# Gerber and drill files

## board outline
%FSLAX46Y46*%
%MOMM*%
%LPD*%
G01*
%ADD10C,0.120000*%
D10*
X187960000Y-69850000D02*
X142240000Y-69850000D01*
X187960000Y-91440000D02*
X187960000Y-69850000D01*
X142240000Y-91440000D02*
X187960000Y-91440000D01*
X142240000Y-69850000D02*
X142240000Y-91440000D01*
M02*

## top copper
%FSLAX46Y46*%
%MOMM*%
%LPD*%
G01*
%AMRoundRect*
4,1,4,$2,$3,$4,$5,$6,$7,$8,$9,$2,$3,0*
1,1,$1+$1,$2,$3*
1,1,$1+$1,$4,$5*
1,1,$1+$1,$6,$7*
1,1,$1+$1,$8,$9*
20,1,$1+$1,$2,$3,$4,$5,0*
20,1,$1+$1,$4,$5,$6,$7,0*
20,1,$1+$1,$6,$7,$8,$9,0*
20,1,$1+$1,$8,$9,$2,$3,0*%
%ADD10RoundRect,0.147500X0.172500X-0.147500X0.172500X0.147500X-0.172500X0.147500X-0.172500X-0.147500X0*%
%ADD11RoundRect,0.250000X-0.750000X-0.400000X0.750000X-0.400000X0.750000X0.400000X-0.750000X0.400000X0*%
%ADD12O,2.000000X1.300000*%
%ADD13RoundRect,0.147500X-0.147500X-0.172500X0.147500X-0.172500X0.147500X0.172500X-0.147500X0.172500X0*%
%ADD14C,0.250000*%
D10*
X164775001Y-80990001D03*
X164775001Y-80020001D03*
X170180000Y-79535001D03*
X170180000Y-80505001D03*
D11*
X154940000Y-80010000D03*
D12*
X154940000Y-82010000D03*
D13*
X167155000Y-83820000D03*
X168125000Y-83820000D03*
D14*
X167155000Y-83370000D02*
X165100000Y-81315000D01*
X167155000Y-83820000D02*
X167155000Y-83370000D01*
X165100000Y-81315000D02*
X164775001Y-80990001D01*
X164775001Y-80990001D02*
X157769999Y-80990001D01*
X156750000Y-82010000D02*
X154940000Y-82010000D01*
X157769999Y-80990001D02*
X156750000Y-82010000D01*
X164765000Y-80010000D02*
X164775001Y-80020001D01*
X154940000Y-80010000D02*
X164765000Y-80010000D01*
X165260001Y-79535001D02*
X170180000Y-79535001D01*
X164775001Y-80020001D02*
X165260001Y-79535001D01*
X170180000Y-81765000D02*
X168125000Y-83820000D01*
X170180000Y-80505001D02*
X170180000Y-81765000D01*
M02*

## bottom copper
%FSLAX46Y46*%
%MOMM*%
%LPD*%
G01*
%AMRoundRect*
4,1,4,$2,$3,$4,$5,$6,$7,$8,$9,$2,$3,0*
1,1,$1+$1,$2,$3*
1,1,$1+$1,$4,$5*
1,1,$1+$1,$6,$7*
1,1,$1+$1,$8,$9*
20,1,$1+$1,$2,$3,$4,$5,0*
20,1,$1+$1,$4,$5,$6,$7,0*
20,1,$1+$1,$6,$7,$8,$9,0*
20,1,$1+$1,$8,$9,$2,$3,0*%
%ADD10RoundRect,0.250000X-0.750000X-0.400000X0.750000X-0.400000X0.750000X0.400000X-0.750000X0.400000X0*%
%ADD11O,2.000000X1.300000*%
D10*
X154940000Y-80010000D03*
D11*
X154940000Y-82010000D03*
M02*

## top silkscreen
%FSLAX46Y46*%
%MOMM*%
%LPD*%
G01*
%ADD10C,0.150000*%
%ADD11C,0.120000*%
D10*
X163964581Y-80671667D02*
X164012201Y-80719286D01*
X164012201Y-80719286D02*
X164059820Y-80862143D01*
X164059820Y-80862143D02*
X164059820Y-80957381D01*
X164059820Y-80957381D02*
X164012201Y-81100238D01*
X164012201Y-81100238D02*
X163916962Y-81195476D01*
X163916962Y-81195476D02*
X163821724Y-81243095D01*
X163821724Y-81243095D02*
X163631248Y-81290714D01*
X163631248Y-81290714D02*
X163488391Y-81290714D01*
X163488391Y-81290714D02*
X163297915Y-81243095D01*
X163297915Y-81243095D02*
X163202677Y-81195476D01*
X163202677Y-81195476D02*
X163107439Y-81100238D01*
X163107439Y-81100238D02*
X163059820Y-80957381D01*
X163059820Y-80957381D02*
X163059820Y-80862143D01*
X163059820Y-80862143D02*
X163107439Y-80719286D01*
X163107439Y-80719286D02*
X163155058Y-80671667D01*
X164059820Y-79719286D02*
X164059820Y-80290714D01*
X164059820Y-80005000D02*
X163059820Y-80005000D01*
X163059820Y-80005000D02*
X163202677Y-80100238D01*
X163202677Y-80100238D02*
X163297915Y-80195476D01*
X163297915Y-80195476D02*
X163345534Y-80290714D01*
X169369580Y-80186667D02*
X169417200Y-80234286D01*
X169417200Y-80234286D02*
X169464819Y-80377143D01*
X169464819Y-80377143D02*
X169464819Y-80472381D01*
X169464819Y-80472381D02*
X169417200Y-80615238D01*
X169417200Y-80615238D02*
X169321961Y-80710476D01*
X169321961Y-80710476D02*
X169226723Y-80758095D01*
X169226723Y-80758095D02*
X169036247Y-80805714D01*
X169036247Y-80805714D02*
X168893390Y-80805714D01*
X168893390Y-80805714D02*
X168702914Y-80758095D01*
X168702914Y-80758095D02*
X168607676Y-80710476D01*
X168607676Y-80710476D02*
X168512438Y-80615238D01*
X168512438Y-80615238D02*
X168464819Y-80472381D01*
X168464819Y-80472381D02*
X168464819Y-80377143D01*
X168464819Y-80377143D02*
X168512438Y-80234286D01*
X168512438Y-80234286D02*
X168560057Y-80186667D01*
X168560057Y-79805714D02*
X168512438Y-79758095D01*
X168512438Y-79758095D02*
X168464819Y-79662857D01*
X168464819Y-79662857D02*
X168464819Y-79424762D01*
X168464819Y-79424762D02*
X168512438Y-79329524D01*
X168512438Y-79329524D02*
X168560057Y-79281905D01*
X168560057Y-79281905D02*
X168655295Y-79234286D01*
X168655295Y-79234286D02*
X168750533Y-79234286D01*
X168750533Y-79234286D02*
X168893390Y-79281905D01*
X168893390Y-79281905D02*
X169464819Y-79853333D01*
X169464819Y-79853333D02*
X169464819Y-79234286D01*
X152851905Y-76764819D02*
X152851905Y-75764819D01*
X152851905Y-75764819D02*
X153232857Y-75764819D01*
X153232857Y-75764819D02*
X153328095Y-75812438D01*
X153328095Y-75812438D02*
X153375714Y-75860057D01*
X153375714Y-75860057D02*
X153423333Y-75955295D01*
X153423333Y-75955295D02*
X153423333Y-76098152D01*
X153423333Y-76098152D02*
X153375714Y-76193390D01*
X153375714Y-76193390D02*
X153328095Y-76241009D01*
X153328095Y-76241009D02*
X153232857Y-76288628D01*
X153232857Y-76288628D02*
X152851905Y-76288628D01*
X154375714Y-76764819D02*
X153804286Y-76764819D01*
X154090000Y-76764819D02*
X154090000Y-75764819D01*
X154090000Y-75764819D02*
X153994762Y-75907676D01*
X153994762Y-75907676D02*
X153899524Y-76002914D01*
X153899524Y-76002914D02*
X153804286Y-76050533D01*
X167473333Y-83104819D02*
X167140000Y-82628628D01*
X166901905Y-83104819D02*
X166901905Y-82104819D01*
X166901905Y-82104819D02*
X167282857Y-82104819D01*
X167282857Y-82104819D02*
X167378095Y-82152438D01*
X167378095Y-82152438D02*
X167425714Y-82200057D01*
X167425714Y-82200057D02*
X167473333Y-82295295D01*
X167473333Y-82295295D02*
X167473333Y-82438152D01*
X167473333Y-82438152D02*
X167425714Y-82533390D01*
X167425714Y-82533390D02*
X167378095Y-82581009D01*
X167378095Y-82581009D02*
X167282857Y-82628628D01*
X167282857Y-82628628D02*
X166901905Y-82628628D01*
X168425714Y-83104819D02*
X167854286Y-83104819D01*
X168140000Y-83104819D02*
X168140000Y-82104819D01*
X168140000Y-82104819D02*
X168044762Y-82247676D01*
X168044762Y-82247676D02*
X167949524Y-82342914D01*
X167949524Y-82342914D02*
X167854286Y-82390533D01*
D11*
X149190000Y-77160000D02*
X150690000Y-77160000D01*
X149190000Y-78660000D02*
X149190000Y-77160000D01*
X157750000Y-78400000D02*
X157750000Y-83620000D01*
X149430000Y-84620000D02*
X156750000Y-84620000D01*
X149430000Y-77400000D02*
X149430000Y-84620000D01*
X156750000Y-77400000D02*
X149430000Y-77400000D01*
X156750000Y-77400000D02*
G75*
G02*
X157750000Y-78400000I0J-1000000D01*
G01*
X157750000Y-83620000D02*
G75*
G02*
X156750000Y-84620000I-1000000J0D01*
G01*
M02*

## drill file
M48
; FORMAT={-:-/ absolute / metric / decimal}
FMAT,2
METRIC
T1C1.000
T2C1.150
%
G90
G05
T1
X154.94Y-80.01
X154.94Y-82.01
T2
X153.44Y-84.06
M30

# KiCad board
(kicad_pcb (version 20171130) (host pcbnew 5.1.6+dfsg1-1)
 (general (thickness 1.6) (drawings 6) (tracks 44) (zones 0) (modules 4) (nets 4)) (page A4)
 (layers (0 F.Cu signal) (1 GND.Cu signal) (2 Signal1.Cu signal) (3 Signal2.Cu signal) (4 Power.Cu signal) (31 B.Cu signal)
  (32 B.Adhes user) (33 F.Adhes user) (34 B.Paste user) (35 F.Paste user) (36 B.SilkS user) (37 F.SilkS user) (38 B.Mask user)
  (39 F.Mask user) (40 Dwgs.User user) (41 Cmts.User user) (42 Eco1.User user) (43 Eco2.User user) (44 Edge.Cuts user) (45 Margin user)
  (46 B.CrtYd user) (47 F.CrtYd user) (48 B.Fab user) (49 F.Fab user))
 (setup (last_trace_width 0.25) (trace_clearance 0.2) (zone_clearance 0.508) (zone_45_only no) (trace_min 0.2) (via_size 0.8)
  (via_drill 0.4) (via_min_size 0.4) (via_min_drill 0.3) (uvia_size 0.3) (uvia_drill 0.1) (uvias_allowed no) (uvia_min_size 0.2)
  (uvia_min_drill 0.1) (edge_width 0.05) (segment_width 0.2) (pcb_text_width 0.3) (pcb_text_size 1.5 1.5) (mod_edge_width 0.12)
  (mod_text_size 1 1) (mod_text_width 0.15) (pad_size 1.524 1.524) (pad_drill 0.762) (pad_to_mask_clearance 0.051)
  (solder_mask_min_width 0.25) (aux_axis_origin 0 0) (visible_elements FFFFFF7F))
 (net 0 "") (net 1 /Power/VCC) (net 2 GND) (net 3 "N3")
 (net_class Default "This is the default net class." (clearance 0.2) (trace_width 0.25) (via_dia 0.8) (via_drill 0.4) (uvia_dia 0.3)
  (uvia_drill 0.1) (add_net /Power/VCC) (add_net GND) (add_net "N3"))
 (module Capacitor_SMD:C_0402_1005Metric (layer F.Cu) (at 164.775001 80.505001 90)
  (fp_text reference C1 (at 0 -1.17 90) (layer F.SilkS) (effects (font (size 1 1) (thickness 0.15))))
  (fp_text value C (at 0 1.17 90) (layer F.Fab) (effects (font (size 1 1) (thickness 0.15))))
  (pad 1 smd roundrect (at -0.485 0 90) (size 0.59 0.64) (layers F.Cu F.Paste F.Mask) (roundrect_rratio 0.25) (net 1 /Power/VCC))
  (pad 2 smd roundrect (at 0.485 0 90) (size 0.59 0.64) (layers F.Cu F.Paste F.Mask) (roundrect_rratio 0.25) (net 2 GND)))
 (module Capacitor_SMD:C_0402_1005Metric (layer F.Cu) (at 170.18 80.020001 90)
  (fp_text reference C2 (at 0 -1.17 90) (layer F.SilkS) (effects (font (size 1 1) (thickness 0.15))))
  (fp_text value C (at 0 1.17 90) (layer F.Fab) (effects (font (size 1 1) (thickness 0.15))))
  (pad 2 smd roundrect (at 0.485 0 90) (size 0.59 0.64) (layers F.Cu F.Paste F.Mask) (roundrect_rratio 0.25) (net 2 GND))
  (pad 1 smd roundrect (at -0.485 0 90) (size 0.59 0.64) (layers F.Cu F.Paste F.Mask) (roundrect_rratio 0.25) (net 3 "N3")))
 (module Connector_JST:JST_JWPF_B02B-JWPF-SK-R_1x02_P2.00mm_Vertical (layer F.Cu) (at 154.94 80.01)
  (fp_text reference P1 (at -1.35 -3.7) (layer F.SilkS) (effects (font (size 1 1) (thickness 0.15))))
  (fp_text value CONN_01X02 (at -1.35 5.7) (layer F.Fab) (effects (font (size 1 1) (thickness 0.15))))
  (fp_line (start -5.75 -2.85) (end -4.25 -2.85) (layer F.SilkS) (width 0.12))
  (fp_line (start -5.75 -1.35) (end -5.75 -2.85) (layer F.SilkS) (width 0.12))
  (fp_line (start 2.81 -1.61) (end 2.81 3.61) (layer F.SilkS) (width 0.12))
  (fp_line (start -5.51 4.61) (end 1.81 4.61) (layer F.SilkS) (width 0.12))
  (fp_line (start -5.51 -2.61) (end -5.51 4.61) (layer F.SilkS) (width 0.12))
  (fp_line (start 1.81 -2.61) (end -5.51 -2.61) (layer F.SilkS) (width 0.12))
  (fp_arc (start 1.81 -1.61) (end 1.81 -2.61) (angle 90) (layer F.SilkS) (width 0.12))
  (fp_arc (start 1.81 3.61) (end 2.81 3.61) (angle 90) (layer F.SilkS) (width 0.12))
  (pad 1 thru_hole roundrect (at 0 0) (size 2 1.3) (drill 1) (layers *.Cu *.Mask) (roundrect_rratio 0.192308) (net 2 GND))
  (pad 2 thru_hole oval (at 0 2) (size 2 1.3) (drill 1) (layers *.Cu *.Mask) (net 1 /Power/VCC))
  (pad "" np_thru_hole circle (at -1.5 4.05) (size 1.15 1.15) (drill 1.15) (layers *.Cu *.Mask)))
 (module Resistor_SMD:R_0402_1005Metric (layer F.Cu) (at 167.64 83.82)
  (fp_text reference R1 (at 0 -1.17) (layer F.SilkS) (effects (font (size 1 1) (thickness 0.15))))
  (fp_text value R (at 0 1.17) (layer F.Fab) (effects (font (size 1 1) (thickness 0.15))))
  (pad 1 smd roundrect (at -0.485 0) (size 0.59 0.64) (layers F.Cu F.Paste F.Mask) (roundrect_rratio 0.25) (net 1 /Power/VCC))
  (pad 2 smd roundrect (at 0.485 0) (size 0.59 0.64) (layers F.Cu F.Paste F.Mask) (roundrect_rratio 0.25) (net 3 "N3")))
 (gr_line (start 187.96 69.85) (end 142.24 69.85) (layer Edge.Cuts) (width 0.12))
 (gr_line (start 187.96 91.44) (end 187.96 69.85) (layer Edge.Cuts) (width 0.12))
 (gr_line (start 142.24 91.44) (end 187.96 91.44) (layer Edge.Cuts) (width 0.12))
 (gr_line (start 142.24 69.85) (end 142.24 91.44) (layer Edge.Cuts) (width 0.12))
 (segment (start 160 73) (end 180 73) (width 0.25) (layer GND.Cu) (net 2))
 (segment (start 180 73) (end 180 88) (width 0.25) (layer GND.Cu) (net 2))
 (segment (start 180 88) (end 160 88) (width 0.25) (layer Signal1.Cu) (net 1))
 (segment (start 161 87) (end 179 87) (width 0.25) (layer Signal2.Cu) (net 2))
 (segment (start 179 87) (end 179 74) (width 0.25) (layer Signal2.Cu) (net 2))
 (segment (start 161 74) (end 179 74) (width 0.25) (layer Power.Cu) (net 1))
 (segment (start 179 74) (end 160.995 74) (width 0.25) (layer Signal2.Cu) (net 2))
 (segment (start 160.995 74) (end 161 74.005) (width 0.25) (layer Signal2.Cu) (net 2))
 (segment (start 180 88) (end 160.009 88) (width 0.25) (layer GND.Cu) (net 2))
 (segment (start 160.009 88) (end 160 87.991) (width 0.25) (layer GND.Cu) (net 2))
 (segment (start 167.155 83.37) (end 165.1 81.315) (width 0.25) (layer F.Cu) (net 1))
 (segment (start 167.155 83.82) (end 167.155 83.37) (width 0.25) (layer F.Cu) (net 1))
 (segment (start 165.1 81.315) (end 164.775001 80.990001) (width 0.25) (layer F.Cu) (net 1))
 (segment (start 164.775001 80.990001) (end 157.769999 80.990001) (width 0.25) (layer F.Cu) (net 1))
 (segment (start 156.75 82.01) (end 154.94 82.01) (width 0.25) (layer F.Cu) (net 1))
 (segment (start 157.769999 80.990001) (end 156.75 82.01) (width 0.25) (layer F.Cu) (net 1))
 (segment (start 159.9226 82.01) (end 160 82.0874) (width 0.25) (layer Signal1.Cu) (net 1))
 (segment (start 154.94 82.01) (end 159.9226 82.01) (width 0.25) (layer Signal1.Cu) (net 1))
 (segment (start 160 82.0874) (end 160 73) (width 0.25) (layer Signal1.Cu) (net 1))
 (segment (start 160 88) (end 160 82.0874) (width 0.25) (layer Signal1.Cu) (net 1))
 (segment (start 180 88) (end 180 73.0152) (width 0.25) (layer Signal1.Cu) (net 1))
 (segment (start 179.9848 73) (end 160 73) (width 0.25) (layer Signal1.Cu) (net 1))
 (segment (start 180 73.0152) (end 179.9848 73) (width 0.25) (layer Signal1.Cu) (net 1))
 (segment (start 160.9786 82.01) (end 161 82.0314) (width 0.25) (layer Power.Cu) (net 1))
 (segment (start 154.94 82.01) (end 160.9786 82.01) (width 0.25) (layer Power.Cu) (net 1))
 (segment (start 161 82.0314) (end 161 87) (width 0.25) (layer Power.Cu) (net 1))
 (segment (start 161 74) (end 161 82.0314) (width 0.25) (layer Power.Cu) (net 1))
 (segment (start 161 87) (end 178.9888 87) (width 0.25) (layer Power.Cu) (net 1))
 (segment (start 179 86.9888) (end 179 74) (width 0.25) (layer Power.Cu) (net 1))
 (segment (start 178.9888 87) (end 179 86.9888) (width 0.25) (layer Power.Cu) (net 1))
 (segment (start 164.765 80.01) (end 164.775001 80.020001) (width 0.25) (layer F.Cu) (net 2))
 (segment (start 154.94 80.01) (end 164.765 80.01) (width 0.25) (layer F.Cu) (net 2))
 (segment (start 165.260001 79.535001) (end 170.18 79.535001) (width 0.25) (layer F.Cu) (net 2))
 (segment (start 164.775001 80.020001) (end 165.260001 79.535001) (width 0.25) (layer F.Cu) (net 2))
 (segment (start 154.9708 79.9792) (end 154.94 80.01) (width 0.25) (layer GND.Cu) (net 2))
 (segment (start 160 79.9792) (end 154.9708 79.9792) (width 0.25) (layer GND.Cu) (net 2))
 (segment (start 160 87.991) (end 160 79.9792) (width 0.25) (layer GND.Cu) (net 2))
 (segment (start 160 79.9792) (end 160 73) (width 0.25) (layer GND.Cu) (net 2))
 (segment (start 160.9852 80.01) (end 161 80.0248) (width 0.25) (layer Signal2.Cu) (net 2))
 (segment (start 154.94 80.01) (end 160.9852 80.01) (width 0.25) (layer Signal2.Cu) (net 2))
 (segment (start 161 80.0248) (end 161 87) (width 0.25) (layer Signal2.Cu) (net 2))
 (segment (start 161 74.005) (end 161 80.0248) (width 0.25) (layer Signal2.Cu) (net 2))
 (segment (start 170.18 81.765) (end 168.125 83.82) (width 0.25) (layer F.Cu) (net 3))
 (segment (start 170.18 80.505001) (end 170.18 81.765) (width 0.25) (layer F.Cu) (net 3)))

